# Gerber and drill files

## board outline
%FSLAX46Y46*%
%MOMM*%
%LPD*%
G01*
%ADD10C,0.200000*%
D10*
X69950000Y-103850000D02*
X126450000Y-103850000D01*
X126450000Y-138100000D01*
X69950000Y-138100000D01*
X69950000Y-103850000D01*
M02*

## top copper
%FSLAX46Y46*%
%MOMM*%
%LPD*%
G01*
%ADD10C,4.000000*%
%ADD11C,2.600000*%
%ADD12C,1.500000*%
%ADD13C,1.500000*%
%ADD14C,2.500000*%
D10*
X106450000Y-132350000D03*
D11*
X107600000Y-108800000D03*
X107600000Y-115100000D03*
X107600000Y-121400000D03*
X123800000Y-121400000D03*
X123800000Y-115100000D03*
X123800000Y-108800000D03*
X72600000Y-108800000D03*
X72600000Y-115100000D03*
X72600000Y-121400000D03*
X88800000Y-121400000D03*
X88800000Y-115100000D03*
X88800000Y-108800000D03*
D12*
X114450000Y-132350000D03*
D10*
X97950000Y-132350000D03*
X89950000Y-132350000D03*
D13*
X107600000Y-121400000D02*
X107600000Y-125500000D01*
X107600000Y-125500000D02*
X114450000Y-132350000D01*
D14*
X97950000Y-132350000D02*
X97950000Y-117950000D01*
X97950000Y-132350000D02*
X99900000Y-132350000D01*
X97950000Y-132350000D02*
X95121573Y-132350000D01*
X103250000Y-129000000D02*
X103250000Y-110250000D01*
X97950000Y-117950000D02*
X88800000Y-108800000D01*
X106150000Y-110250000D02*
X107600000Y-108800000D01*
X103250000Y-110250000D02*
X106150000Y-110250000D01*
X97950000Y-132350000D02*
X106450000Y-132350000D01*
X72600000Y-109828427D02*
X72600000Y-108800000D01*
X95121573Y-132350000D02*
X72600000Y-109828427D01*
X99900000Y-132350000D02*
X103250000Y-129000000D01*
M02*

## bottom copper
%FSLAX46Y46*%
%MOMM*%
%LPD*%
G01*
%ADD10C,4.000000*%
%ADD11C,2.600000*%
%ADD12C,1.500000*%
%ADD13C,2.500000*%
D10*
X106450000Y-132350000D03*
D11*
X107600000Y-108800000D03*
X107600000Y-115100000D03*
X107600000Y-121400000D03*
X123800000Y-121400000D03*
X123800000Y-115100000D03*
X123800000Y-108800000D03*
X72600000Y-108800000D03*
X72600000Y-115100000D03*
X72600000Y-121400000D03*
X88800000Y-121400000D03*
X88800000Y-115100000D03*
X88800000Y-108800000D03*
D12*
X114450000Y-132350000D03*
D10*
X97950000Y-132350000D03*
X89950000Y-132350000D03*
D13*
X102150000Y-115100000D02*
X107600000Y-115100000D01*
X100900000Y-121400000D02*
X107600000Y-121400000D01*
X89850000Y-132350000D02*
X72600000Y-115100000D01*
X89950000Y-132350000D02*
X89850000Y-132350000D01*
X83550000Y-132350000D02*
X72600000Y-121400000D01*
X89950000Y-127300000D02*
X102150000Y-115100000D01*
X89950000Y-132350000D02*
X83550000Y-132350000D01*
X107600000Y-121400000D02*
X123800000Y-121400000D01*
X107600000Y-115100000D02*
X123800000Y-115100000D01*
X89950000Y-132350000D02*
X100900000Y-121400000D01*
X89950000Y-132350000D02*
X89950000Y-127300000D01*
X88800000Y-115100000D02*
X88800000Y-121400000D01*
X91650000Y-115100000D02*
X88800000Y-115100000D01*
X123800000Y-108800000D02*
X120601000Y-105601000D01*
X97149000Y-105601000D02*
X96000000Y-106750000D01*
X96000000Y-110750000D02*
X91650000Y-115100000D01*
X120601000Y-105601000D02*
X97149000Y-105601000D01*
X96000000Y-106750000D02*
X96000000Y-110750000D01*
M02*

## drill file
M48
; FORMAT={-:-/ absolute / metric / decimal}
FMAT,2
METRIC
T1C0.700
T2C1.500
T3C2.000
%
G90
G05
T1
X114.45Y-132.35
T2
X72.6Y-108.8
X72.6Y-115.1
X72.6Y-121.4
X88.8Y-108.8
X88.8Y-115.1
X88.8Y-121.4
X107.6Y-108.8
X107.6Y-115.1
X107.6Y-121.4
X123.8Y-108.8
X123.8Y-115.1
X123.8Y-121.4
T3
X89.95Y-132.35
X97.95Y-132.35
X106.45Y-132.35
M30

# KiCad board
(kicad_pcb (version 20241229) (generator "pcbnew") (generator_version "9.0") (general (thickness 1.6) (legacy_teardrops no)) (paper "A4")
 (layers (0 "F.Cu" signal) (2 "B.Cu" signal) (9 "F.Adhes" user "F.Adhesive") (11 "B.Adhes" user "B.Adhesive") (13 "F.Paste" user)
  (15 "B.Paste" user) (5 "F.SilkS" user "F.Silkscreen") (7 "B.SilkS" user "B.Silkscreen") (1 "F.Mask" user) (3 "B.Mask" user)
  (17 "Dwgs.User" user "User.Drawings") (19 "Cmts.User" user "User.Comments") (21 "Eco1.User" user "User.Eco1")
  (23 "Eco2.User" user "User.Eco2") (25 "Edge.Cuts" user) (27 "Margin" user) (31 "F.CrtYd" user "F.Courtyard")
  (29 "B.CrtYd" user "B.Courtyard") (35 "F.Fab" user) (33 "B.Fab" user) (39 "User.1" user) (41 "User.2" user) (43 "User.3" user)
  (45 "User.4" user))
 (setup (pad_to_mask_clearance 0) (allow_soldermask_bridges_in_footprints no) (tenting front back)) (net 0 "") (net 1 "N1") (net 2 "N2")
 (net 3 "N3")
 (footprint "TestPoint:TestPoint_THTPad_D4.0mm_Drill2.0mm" (layer "F.Cu") (at 106.45 132.35)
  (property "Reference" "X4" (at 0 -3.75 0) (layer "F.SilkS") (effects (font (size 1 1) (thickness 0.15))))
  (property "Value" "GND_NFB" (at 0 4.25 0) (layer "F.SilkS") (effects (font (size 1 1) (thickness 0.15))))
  (pad "1" thru_hole circle (at 0 0) (size 4 4) (drill 2) (layers "*.Cu" "*.Mask") (remove_unused_layers no) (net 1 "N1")))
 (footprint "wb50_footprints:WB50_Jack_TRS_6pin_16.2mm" (layer "F.Cu") (at 115.7 115.1 180)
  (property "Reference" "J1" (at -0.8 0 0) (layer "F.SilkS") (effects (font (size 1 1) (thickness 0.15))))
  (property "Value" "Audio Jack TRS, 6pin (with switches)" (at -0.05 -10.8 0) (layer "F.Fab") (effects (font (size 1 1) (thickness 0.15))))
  (pad "1" thru_hole circle (at 8.1 6.3 90) (size 2.6 2.6) (drill 1.5) (layers "*.Cu" "*.Mask") (remove_unused_layers no) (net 1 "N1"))
  (pad "2" thru_hole circle (at 8.1 0 90) (size 2.6 2.6) (drill 1.5) (layers "*.Cu" "*.Mask") (remove_unused_layers no) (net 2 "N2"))
  (pad "3" thru_hole circle (at 8.1 -6.3 90) (size 2.6 2.6) (drill 1.5) (layers "*.Cu" "*.Mask") (remove_unused_layers no) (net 2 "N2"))
  (pad "4" thru_hole circle (at -8.1 -6.3 90) (size 2.6 2.6) (drill 1.5) (layers "*.Cu" "*.Mask") (remove_unused_layers no) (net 2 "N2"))
  (pad "5" thru_hole circle (at -8.1 0 90) (size 2.6 2.6) (drill 1.5) (layers "*.Cu" "*.Mask") (remove_unused_layers no) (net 2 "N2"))
  (pad "6" thru_hole circle (at -8.1 6.3 90) (size 2.6 2.6) (drill 1.5) (layers "*.Cu" "*.Mask") (remove_unused_layers no) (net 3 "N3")))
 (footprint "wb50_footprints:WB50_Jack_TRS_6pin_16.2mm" (layer "F.Cu") (at 80.7 115.1 180)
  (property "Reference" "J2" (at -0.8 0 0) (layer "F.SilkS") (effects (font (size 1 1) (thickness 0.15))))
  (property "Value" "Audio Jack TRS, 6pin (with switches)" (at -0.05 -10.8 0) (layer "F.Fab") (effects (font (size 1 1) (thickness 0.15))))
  (pad "1" thru_hole circle (at 8.1 6.3 90) (size 2.6 2.6) (drill 1.5) (layers "*.Cu" "*.Mask") (remove_unused_layers no) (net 1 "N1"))
  (pad "2" thru_hole circle (at 8.1 0 90) (size 2.6 2.6) (drill 1.5) (layers "*.Cu" "*.Mask") (remove_unused_layers no) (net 2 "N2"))
  (pad "3" thru_hole circle (at 8.1 -6.3 90) (size 2.6 2.6) (drill 1.5) (layers "*.Cu" "*.Mask") (remove_unused_layers no) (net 2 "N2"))
  (pad "4" thru_hole circle (at -8.1 -6.3 90) (size 2.6 2.6) (drill 1.5) (layers "*.Cu" "*.Mask") (remove_unused_layers no) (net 3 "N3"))
  (pad "5" thru_hole circle (at -8.1 0 90) (size 2.6 2.6) (drill 1.5) (layers "*.Cu" "*.Mask") (remove_unused_layers no) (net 3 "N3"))
  (pad "6" thru_hole circle (at -8.1 6.3 90) (size 2.6 2.6) (drill 1.5) (layers "*.Cu" "*.Mask") (remove_unused_layers no) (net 1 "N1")))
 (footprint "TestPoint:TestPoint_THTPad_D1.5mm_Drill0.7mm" (layer "F.Cu") (at 114.45 132.35)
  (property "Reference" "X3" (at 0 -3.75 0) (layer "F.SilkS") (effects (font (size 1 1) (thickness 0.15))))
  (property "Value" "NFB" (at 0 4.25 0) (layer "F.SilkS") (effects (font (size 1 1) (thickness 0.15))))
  (pad "1" thru_hole circle (at 0 0) (size 1.5 1.5) (drill 0.7) (layers "*.Cu" "*.Mask") (remove_unused_layers no) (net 2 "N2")))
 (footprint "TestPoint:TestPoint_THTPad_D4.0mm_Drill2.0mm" (layer "F.Cu") (at 97.95 132.35)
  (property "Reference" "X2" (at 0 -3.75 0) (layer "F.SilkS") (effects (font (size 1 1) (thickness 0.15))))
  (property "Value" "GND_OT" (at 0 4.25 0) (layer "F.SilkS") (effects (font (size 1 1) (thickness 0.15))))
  (pad "1" thru_hole circle (at 0 0) (size 4 4) (drill 2) (layers "*.Cu" "*.Mask") (remove_unused_layers no) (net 1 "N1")))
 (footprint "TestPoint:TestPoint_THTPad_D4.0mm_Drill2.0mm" (layer "F.Cu") (at 89.95 132.35)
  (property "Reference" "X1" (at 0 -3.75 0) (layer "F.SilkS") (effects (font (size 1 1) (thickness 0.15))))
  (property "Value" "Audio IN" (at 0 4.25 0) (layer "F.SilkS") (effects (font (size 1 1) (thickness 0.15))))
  (pad "1" thru_hole circle (at 0 0) (size 4 4) (drill 2) (layers "*.Cu" "*.Mask") (remove_unused_layers no) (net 2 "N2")))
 (gr_rect (start 69.95 103.85) (end 126.45 138.1) (stroke (width 0.2) (type default)) (fill no) (layer "Edge.Cuts"))
 (segment (start 107.6 121.4) (end 107.6 125.5) (width 1.5) (layer "F.Cu") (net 2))
 (segment (start 107.6 125.5) (end 114.45 132.35) (width 1.5) (layer "F.Cu") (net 2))
 (segment (start 102.15 115.1) (end 107.6 115.1) (width 2.5) (layer "B.Cu") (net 2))
 (segment (start 100.9 121.4) (end 107.6 121.4) (width 2.5) (layer "B.Cu") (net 2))
 (segment (start 89.85 132.35) (end 72.6 115.1) (width 2.5) (layer "B.Cu") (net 2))
 (segment (start 89.95 132.35) (end 89.85 132.35) (width 2.5) (layer "B.Cu") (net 2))
 (segment (start 83.55 132.35) (end 72.6 121.4) (width 2.5) (layer "B.Cu") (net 2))
 (segment (start 89.95 127.3) (end 102.15 115.1) (width 2.5) (layer "B.Cu") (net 2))
 (segment (start 89.95 132.35) (end 83.55 132.35) (width 2.5) (layer "B.Cu") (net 2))
 (segment (start 107.6 121.4) (end 123.8 121.4) (width 2.5) (layer "B.Cu") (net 2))
 (segment (start 107.6 115.1) (end 123.8 115.1) (width 2.5) (layer "B.Cu") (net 2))
 (segment (start 89.95 132.35) (end 100.9 121.4) (width 2.5) (layer "B.Cu") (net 2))
 (segment (start 89.95 132.35) (end 89.95 127.3) (width 2.5) (layer "B.Cu") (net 2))
 (segment (start 88.8 115.1) (end 88.8 121.4) (width 2.5) (layer "B.Cu") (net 3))
 (segment (start 91.65 115.1) (end 88.8 115.1) (width 2.5) (layer "B.Cu") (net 3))
 (segment (start 123.8 108.8) (end 120.601 105.601) (width 2.5) (layer "B.Cu") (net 3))
 (segment (start 97.149 105.601) (end 96 106.75) (width 2.5) (layer "B.Cu") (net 3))
 (segment (start 96 110.75) (end 91.65 115.1) (width 2.5) (layer "B.Cu") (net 3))
 (segment (start 120.601 105.601) (end 97.149 105.601) (width 2.5) (layer "B.Cu") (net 3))
 (segment (start 96 106.75) (end 96 110.75) (width 2.5) (layer "B.Cu") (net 3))
 (segment (start 97.95 132.35) (end 97.95 117.95) (width 2.5) (layer "F.Cu") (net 1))
 (segment (start 97.95 132.35) (end 99.9 132.35) (width 2.5) (layer "F.Cu") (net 1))
 (segment (start 97.95 132.35) (end 95.121573 132.35) (width 2.5) (layer "F.Cu") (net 1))
 (segment (start 103.25 129) (end 103.25 110.25) (width 2.5) (layer "F.Cu") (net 1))
 (segment (start 97.95 117.95) (end 88.8 108.8) (width 2.5) (layer "F.Cu") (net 1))
 (segment (start 106.15 110.25) (end 107.6 108.8) (width 2.5) (layer "F.Cu") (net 1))
 (segment (start 103.25 110.25) (end 106.15 110.25) (width 2.5) (layer "F.Cu") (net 1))
 (segment (start 97.95 132.35) (end 106.45 132.35) (width 2.5) (layer "F.Cu") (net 1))
 (segment (start 72.6 109.828427) (end 72.6 108.8) (width 2.5) (layer "F.Cu") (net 1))
 (segment (start 95.121573 132.35) (end 72.6 109.828427) (width 2.5) (layer "F.Cu") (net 1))
 (segment (start 99.9 132.35) (end 103.25 129) (width 2.5) (layer "F.Cu") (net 1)))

